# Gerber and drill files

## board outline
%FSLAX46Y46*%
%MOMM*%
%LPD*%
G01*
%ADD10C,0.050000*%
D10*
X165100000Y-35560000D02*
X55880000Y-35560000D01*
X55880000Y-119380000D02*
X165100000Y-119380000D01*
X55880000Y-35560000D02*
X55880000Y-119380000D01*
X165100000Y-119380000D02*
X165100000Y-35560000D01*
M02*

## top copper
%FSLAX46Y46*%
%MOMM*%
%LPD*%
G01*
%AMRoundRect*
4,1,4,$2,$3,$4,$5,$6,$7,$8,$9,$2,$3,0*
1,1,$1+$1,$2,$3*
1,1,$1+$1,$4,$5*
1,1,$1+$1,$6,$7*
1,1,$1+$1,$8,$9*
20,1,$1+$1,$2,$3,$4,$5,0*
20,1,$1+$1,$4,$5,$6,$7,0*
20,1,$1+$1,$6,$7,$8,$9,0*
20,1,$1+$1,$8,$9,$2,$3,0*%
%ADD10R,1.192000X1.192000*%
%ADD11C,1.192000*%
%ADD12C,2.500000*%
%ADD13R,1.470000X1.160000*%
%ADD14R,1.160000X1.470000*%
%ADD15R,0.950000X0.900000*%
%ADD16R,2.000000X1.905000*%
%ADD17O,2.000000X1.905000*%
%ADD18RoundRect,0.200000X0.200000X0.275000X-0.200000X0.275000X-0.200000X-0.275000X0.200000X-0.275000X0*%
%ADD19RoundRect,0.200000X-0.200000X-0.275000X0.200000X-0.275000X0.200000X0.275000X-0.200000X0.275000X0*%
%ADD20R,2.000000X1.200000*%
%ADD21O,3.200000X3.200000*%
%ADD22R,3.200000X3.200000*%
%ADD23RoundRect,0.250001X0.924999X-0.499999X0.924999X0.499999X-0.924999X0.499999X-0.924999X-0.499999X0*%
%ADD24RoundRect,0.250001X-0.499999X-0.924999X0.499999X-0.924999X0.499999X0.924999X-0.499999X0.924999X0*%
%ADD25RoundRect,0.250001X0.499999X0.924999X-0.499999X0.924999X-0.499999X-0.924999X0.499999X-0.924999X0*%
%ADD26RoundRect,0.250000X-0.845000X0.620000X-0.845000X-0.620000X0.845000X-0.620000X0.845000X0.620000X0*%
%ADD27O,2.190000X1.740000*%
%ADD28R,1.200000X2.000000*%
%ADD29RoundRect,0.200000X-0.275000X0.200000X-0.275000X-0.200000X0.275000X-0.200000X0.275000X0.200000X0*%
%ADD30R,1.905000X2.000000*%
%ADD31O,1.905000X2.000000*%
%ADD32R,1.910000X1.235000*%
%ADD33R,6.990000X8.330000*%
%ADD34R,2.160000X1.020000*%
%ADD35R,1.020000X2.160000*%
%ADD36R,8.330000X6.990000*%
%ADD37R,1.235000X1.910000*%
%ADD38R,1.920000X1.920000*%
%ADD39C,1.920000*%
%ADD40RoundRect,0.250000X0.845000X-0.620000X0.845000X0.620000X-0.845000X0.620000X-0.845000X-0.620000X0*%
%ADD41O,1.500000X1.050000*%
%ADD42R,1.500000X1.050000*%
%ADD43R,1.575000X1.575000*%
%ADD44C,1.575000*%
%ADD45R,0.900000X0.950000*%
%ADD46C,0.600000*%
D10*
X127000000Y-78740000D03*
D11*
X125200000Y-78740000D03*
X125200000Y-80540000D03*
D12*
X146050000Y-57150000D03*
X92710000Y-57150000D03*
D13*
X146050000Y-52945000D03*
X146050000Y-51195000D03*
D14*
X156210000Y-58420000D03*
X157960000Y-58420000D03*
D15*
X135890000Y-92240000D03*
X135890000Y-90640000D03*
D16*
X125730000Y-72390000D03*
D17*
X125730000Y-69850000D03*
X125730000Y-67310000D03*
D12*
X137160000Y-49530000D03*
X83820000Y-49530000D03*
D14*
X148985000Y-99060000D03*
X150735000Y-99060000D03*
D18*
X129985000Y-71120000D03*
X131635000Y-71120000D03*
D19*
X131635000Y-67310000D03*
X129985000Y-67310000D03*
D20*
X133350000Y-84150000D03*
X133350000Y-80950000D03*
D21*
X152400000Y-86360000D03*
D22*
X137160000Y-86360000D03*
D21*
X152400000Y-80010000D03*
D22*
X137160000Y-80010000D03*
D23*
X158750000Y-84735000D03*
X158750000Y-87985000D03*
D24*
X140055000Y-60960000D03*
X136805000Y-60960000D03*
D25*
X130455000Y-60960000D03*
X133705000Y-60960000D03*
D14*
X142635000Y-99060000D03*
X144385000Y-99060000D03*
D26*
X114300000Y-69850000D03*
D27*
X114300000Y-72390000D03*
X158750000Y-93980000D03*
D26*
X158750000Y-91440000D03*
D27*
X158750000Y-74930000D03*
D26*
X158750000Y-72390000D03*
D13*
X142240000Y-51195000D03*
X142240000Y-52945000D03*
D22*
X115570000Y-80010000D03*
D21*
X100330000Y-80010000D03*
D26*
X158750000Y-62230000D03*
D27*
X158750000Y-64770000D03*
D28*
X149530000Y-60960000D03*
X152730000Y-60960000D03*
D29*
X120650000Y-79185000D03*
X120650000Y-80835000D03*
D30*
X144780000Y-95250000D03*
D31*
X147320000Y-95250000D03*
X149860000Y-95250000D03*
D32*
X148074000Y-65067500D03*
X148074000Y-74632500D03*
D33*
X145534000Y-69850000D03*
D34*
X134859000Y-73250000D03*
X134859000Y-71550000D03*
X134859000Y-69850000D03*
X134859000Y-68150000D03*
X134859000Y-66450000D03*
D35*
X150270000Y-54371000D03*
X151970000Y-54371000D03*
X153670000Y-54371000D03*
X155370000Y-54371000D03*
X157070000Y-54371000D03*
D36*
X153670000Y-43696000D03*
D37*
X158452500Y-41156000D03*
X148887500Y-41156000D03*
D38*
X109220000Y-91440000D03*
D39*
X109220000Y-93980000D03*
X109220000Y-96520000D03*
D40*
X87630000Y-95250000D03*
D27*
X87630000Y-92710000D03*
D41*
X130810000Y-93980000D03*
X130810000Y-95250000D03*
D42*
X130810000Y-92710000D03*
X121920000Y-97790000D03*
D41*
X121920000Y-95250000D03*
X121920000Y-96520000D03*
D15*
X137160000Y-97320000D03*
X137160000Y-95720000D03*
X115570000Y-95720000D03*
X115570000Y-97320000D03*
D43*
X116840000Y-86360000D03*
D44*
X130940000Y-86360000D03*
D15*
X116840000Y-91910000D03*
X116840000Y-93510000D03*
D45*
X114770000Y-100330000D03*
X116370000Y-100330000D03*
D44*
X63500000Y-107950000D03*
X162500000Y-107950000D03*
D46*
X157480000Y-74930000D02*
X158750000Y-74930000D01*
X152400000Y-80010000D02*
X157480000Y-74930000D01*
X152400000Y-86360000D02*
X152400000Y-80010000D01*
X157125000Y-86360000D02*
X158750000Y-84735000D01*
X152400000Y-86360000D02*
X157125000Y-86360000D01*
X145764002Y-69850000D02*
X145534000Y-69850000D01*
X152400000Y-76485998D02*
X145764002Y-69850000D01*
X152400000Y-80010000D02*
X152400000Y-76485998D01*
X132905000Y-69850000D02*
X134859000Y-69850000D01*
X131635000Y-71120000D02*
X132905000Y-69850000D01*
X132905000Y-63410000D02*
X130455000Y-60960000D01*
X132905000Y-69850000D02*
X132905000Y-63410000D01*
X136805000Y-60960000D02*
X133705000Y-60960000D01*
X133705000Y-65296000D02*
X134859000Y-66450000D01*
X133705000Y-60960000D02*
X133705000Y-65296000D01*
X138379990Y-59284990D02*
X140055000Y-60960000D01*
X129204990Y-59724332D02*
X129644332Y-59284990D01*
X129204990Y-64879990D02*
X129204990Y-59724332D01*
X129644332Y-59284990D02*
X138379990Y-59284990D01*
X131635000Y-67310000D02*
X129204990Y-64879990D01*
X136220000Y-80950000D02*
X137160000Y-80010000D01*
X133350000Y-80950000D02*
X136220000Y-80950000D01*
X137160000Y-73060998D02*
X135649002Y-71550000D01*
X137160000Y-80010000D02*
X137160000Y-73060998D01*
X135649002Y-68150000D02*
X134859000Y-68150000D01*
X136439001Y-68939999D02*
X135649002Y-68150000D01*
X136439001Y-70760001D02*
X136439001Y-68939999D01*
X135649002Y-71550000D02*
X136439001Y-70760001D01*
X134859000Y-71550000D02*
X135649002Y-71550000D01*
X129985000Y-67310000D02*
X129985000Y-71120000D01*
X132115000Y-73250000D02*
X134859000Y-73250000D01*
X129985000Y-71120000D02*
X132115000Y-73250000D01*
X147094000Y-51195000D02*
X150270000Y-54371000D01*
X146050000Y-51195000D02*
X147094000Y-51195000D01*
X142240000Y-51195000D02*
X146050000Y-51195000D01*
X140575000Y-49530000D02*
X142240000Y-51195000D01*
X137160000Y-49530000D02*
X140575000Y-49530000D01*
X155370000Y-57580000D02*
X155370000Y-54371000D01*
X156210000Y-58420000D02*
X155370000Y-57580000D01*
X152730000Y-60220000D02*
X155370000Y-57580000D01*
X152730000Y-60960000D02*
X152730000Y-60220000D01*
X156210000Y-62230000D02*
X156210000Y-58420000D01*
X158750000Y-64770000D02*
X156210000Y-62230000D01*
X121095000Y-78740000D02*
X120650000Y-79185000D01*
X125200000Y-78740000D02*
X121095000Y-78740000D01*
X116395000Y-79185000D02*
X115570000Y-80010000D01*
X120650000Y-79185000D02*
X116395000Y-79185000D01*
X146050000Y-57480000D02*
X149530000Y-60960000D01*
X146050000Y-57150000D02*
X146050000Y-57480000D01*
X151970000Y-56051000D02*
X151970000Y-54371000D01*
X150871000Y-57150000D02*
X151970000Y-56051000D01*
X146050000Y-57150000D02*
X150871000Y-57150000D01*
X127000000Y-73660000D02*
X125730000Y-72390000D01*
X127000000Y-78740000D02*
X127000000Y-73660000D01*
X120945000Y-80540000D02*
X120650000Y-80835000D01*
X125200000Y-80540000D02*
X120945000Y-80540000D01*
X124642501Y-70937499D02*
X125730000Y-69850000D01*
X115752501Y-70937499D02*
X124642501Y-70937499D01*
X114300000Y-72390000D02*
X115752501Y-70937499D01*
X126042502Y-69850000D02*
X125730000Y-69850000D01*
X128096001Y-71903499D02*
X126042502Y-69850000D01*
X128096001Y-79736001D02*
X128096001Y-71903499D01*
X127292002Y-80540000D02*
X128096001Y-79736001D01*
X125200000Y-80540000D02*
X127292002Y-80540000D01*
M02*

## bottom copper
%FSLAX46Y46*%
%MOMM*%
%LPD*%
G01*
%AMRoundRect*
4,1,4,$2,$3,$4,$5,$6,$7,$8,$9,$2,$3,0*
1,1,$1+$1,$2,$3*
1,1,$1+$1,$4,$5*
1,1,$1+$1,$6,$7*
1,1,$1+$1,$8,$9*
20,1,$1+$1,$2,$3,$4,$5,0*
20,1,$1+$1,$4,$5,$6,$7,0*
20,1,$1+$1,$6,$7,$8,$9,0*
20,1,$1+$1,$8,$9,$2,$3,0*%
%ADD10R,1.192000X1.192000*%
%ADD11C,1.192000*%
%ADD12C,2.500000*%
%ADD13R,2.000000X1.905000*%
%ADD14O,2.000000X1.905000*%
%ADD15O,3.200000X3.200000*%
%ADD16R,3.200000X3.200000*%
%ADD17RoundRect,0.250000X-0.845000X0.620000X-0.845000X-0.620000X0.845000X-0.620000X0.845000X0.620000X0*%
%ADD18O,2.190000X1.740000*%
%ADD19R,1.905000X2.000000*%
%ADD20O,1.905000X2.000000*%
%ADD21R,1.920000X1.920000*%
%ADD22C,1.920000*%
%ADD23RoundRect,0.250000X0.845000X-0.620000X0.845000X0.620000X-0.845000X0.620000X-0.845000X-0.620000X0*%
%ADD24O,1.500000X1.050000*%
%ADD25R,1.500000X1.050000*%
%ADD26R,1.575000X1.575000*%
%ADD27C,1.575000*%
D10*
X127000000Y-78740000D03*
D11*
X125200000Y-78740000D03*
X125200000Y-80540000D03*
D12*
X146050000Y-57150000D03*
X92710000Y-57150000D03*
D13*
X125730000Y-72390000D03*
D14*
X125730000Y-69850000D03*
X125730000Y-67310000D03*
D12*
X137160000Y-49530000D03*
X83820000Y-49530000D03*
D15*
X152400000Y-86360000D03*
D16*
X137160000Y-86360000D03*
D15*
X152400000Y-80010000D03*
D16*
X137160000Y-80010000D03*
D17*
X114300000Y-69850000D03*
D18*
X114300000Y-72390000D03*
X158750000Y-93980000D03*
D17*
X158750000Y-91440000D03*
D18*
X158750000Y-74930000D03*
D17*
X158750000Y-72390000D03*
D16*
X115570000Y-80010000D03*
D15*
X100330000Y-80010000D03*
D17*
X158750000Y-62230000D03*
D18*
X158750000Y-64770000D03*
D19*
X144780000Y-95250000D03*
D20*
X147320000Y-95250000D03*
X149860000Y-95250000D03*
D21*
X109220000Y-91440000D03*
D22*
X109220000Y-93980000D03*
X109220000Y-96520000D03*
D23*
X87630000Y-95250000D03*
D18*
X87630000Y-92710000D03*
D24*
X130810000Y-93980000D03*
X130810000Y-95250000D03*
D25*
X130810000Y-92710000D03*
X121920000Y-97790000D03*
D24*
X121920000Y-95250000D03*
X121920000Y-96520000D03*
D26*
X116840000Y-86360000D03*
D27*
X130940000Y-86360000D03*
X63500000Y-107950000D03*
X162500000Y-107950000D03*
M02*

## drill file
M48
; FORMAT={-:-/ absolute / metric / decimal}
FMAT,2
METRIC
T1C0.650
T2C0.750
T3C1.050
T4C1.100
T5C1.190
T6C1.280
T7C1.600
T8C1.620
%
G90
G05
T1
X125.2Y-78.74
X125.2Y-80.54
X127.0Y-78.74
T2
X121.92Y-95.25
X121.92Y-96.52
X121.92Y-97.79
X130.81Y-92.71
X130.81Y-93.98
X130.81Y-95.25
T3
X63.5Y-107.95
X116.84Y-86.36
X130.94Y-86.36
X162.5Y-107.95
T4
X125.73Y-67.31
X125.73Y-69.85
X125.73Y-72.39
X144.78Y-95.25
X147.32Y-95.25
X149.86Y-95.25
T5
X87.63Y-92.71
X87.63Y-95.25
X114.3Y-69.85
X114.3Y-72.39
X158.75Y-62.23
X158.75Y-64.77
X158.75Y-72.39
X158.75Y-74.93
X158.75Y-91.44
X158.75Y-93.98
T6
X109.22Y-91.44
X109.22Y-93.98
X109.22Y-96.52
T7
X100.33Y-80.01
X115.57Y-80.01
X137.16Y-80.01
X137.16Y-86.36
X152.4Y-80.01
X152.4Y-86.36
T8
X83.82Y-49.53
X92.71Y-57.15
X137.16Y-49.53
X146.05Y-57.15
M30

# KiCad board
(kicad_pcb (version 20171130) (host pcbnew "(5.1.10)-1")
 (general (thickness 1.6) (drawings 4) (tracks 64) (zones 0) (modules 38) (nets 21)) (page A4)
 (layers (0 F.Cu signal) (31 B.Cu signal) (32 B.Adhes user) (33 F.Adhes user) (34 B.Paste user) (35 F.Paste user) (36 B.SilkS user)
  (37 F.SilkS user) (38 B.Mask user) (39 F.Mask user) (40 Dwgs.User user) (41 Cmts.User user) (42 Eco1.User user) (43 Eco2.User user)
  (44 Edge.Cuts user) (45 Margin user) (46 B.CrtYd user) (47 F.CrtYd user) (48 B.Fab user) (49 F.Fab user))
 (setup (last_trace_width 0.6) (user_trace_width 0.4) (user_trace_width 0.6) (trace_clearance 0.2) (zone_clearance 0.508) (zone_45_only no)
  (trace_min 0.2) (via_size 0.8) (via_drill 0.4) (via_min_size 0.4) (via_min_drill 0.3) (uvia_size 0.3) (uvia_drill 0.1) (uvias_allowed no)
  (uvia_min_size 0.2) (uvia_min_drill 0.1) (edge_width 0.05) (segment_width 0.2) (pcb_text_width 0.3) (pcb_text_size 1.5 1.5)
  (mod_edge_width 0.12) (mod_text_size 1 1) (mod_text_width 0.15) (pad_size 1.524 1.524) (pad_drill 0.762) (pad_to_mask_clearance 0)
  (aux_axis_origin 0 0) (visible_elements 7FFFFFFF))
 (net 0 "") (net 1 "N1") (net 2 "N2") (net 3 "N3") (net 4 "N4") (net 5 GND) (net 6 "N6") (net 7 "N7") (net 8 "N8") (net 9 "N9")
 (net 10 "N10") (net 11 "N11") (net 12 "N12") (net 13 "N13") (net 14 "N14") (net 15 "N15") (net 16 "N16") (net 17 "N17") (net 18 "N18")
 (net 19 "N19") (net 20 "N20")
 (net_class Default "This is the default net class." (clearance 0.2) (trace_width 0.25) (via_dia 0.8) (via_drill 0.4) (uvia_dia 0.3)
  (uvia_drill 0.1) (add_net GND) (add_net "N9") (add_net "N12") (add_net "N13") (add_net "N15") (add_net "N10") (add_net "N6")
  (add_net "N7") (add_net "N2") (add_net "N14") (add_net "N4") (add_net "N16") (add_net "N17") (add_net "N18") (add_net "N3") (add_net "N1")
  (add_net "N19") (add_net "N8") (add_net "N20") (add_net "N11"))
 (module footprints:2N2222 (layer F.Cu) (at 127 78.74 180)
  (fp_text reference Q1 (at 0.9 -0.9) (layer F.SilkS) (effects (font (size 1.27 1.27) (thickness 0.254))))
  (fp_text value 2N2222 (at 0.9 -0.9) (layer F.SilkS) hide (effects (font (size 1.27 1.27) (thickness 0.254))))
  (pad 1 thru_hole rect (at 0 0 180) (size 1.192 1.192) (drill 0.65) (layers *.Cu *.Mask) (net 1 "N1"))
  (pad 2 thru_hole circle (at 1.8 0 180) (size 1.192 1.192) (drill 0.65) (layers *.Cu *.Mask) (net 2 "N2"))
  (pad 3 thru_hole circle (at 1.8 -1.8 180) (size 1.192 1.192) (drill 0.65) (layers *.Cu *.Mask) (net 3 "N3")))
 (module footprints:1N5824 (layer F.Cu) (at 119.38 57.15)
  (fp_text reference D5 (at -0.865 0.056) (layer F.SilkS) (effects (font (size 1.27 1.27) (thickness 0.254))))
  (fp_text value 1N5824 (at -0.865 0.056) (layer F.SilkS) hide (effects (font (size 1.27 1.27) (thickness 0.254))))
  (pad 1 thru_hole circle (at 26.67 0) (size 2.5 2.5) (drill 1.62) (layers *.Cu *.Mask) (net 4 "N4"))
  (pad 2 thru_hole circle (at -26.67 0) (size 2.5 2.5) (drill 1.62) (layers *.Cu *.Mask) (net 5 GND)))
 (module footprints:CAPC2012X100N (layer F.Cu) (at 146.05 52.07 270)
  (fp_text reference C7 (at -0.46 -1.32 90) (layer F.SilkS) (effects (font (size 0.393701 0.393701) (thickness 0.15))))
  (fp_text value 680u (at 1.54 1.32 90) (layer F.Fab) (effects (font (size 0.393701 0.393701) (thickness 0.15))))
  (pad 2 smd rect (at 0.875 0 270) (size 1.16 1.47) (layers F.Cu F.Paste F.Mask) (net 5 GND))
  (pad 1 smd rect (at -0.875 0 270) (size 1.16 1.47) (layers F.Cu F.Paste F.Mask) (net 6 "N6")))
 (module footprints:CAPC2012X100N (layer F.Cu) (at 157.085 58.42)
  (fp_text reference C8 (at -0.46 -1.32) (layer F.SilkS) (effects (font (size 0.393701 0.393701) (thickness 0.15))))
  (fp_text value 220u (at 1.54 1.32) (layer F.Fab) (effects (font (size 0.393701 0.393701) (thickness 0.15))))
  (pad 1 smd rect (at -0.875 0) (size 1.16 1.47) (layers F.Cu F.Paste F.Mask) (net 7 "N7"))
  (pad 2 smd rect (at 0.875 0) (size 1.16 1.47) (layers F.Cu F.Paste F.Mask) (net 5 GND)))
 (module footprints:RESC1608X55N (layer F.Cu) (at 135.89 91.44 90)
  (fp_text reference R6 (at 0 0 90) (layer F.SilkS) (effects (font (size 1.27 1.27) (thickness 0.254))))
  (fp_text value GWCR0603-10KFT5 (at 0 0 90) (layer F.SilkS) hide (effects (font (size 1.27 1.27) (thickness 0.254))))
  (pad 1 smd rect (at -0.8 0 90) (size 0.9 0.95) (layers F.Cu F.Paste F.Mask) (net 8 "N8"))
  (pad 2 smd rect (at 0.8 0 90) (size 0.9 0.95) (layers F.Cu F.Paste F.Mask) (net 5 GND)))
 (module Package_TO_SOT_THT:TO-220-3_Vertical (layer F.Cu) (at 125.73 72.39 90)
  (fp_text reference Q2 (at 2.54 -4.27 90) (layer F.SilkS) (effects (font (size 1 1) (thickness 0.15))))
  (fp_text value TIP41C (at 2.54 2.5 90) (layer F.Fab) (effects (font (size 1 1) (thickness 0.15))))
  (pad 1 thru_hole rect (at 0 0 90) (size 1.905 2) (drill 1.1) (layers *.Cu *.Mask) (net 1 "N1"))
  (pad 2 thru_hole oval (at 2.54 0 90) (size 1.905 2) (drill 1.1) (layers *.Cu *.Mask) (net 3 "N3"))
  (pad 3 thru_hole oval (at 5.08 0 90) (size 1.905 2) (drill 1.1) (layers *.Cu *.Mask) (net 6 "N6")))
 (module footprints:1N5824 (layer F.Cu) (at 110.49 49.53 180)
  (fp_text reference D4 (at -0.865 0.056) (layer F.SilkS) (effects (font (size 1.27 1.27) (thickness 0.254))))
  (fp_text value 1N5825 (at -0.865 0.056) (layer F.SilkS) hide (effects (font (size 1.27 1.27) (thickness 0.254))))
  (pad 2 thru_hole circle (at -26.67 0 180) (size 2.5 2.5) (drill 1.62) (layers *.Cu *.Mask) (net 6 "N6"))
  (pad 1 thru_hole circle (at 26.67 0 180) (size 2.5 2.5) (drill 1.62) (layers *.Cu *.Mask) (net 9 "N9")))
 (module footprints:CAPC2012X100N (layer F.Cu) (at 149.86 99.06 180)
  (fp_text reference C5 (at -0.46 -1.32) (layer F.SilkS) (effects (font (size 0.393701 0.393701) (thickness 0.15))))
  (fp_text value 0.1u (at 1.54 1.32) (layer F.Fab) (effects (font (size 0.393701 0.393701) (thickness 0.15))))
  (pad 2 smd rect (at 0.875 0 180) (size 1.16 1.47) (layers F.Cu F.Paste F.Mask) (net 5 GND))
  (pad 1 smd rect (at -0.875 0 180) (size 1.16 1.47) (layers F.Cu F.Paste F.Mask) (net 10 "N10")))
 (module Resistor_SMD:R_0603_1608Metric (layer F.Cu) (at 130.81 71.12 180)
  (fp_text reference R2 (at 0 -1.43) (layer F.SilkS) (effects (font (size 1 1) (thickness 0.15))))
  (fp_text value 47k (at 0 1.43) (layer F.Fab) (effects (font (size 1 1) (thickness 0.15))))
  (pad 2 smd roundrect (at 0.825 0 180) (size 0.8 0.95) (layers F.Cu F.Paste F.Mask) (roundrect_rratio 0.25) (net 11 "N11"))
  (pad 1 smd roundrect (at -0.825 0 180) (size 0.8 0.95) (layers F.Cu F.Paste F.Mask) (roundrect_rratio 0.25) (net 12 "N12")))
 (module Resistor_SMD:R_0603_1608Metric (layer F.Cu) (at 130.81 67.31)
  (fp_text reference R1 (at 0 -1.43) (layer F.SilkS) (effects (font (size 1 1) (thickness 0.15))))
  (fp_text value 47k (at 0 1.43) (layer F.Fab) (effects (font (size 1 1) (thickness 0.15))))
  (pad 2 smd roundrect (at 0.825 0) (size 0.8 0.95) (layers F.Cu F.Paste F.Mask) (roundrect_rratio 0.25) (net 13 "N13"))
  (pad 1 smd roundrect (at -0.825 0) (size 0.8 0.95) (layers F.Cu F.Paste F.Mask) (roundrect_rratio 0.25) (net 11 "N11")))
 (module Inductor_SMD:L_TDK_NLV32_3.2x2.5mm (layer F.Cu) (at 133.35 82.55 270)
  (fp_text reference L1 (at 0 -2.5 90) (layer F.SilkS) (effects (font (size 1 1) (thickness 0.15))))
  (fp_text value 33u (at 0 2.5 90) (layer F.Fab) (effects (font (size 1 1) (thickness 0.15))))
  (pad 2 smd rect (at 1.6 0 270) (size 1.2 2) (layers F.Cu F.Paste F.Mask) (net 5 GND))
  (pad 1 smd rect (at -1.6 0 270) (size 1.2 2) (layers F.Cu F.Paste F.Mask) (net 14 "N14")))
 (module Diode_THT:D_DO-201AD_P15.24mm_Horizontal (layer F.Cu) (at 137.16 86.36)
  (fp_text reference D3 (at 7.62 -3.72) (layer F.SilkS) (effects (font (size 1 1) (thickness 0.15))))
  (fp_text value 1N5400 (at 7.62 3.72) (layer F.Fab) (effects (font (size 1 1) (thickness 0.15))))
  (pad 2 thru_hole oval (at 15.24 0) (size 3.2 3.2) (drill 1.6) (layers *.Cu *.Mask) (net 12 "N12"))
  (pad 1 thru_hole rect (at 0 0) (size 3.2 3.2) (drill 1.6) (layers *.Cu *.Mask) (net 5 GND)))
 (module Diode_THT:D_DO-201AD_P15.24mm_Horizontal (layer F.Cu) (at 137.16 80.01)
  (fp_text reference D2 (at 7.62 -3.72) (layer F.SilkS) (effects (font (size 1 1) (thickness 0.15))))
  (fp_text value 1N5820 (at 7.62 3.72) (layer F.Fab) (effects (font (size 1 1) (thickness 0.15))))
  (pad 2 thru_hole oval (at 15.24 0) (size 3.2 3.2) (drill 1.6) (layers *.Cu *.Mask) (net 12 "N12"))
  (pad 1 thru_hole rect (at 0 0) (size 3.2 3.2) (drill 1.6) (layers *.Cu *.Mask) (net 14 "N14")))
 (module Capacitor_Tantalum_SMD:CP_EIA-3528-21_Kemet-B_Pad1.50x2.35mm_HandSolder (layer F.Cu) (at 158.75 86.36 90)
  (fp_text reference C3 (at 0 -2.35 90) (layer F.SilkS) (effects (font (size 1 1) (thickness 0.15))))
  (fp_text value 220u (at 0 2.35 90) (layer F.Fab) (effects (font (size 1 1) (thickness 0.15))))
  (pad 2 smd roundrect (at 1.625 0 90) (size 1.5 2.35) (layers F.Cu F.Paste F.Mask) (roundrect_rratio 0.166667) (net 12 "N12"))
  (pad 1 smd roundrect (at -1.625 0 90) (size 1.5 2.35) (layers F.Cu F.Paste F.Mask) (roundrect_rratio 0.166667) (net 5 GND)))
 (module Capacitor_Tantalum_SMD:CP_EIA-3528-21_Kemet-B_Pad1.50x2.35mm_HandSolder (layer F.Cu) (at 138.43 60.96)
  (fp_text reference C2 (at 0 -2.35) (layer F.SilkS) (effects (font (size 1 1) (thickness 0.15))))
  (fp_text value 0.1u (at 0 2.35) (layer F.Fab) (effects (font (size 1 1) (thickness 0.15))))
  (pad 2 smd roundrect (at 1.625 0) (size 1.5 2.35) (layers F.Cu F.Paste F.Mask) (roundrect_rratio 0.166667) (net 13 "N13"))
  (pad 1 smd roundrect (at -1.625 0) (size 1.5 2.35) (layers F.Cu F.Paste F.Mask) (roundrect_rratio 0.166667) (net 9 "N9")))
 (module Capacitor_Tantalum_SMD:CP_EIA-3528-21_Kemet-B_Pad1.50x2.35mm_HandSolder (layer F.Cu) (at 132.08 60.96 180)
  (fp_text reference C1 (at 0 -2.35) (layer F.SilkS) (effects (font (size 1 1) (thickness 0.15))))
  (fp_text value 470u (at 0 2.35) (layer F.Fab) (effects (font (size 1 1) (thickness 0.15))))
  (pad 2 smd roundrect (at 1.625 0 180) (size 1.5 2.35) (layers F.Cu F.Paste F.Mask) (roundrect_rratio 0.166667) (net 12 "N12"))
  (pad 1 smd roundrect (at -1.625 0 180) (size 1.5 2.35) (layers F.Cu F.Paste F.Mask) (roundrect_rratio 0.166667) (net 9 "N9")))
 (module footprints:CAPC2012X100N (layer F.Cu) (at 143.51 99.06)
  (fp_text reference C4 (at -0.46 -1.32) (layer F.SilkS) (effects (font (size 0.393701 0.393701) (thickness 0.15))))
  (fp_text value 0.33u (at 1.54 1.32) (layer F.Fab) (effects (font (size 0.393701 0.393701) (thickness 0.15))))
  (pad 1 smd rect (at -0.875 0) (size 1.16 1.47) (layers F.Cu F.Paste F.Mask) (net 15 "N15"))
  (pad 2 smd rect (at 0.875 0) (size 1.16 1.47) (layers F.Cu F.Paste F.Mask) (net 5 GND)))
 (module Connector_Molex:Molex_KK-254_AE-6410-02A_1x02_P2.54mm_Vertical (layer F.Cu) (at 114.3 69.85 270)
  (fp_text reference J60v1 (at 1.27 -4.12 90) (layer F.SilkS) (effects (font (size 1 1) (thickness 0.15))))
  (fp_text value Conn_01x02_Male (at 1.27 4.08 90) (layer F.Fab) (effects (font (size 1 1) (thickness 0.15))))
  (pad 1 thru_hole roundrect (at 0 0 270) (size 1.74 2.19) (drill 1.19) (layers *.Cu *.Mask) (roundrect_rratio 0.143678) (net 5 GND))
  (pad 2 thru_hole oval (at 2.54 0 270) (size 1.74 2.19) (drill 1.19) (layers *.Cu *.Mask) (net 3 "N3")))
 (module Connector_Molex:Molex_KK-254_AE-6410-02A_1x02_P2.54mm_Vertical (layer F.Cu) (at 158.75 91.44 270)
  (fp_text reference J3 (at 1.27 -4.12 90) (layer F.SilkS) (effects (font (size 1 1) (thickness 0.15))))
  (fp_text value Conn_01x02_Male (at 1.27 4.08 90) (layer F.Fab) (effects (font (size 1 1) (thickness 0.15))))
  (pad 2 thru_hole oval (at 2.54 0 270) (size 1.74 2.19) (drill 1.19) (layers *.Cu *.Mask) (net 10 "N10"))
  (pad 1 thru_hole roundrect (at 0 0 270) (size 1.74 2.19) (drill 1.19) (layers *.Cu *.Mask) (roundrect_rratio 0.143678) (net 5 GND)))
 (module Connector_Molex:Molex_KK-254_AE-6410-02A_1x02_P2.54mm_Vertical (layer F.Cu) (at 158.75 72.39 270)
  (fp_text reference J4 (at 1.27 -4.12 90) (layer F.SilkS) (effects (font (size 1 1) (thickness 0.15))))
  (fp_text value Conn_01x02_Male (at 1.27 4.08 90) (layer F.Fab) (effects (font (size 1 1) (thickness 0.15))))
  (pad 2 thru_hole oval (at 2.54 0 270) (size 1.74 2.19) (drill 1.19) (layers *.Cu *.Mask) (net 12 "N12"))
  (pad 1 thru_hole roundrect (at 0 0 270) (size 1.74 2.19) (drill 1.19) (layers *.Cu *.Mask) (roundrect_rratio 0.143678) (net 5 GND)))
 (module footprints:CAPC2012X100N (layer F.Cu) (at 142.24 52.07 270)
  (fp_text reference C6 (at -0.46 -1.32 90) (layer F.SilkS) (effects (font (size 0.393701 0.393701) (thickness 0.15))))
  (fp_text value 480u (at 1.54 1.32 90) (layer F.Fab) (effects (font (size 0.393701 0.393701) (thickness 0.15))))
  (pad 1 smd rect (at -0.875 0 270) (size 1.16 1.47) (layers F.Cu F.Paste F.Mask) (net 6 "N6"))
  (pad 2 smd rect (at 0.875 0 270) (size 1.16 1.47) (layers F.Cu F.Paste F.Mask) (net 5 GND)))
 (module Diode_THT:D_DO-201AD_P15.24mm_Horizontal (layer F.Cu) (at 115.57 80.01 180)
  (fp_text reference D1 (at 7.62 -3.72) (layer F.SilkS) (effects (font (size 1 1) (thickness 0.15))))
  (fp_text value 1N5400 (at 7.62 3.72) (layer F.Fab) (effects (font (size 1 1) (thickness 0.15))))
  (pad 1 thru_hole rect (at 0 0 180) (size 3.2 3.2) (drill 1.6) (layers *.Cu *.Mask) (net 2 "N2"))
  (pad 2 thru_hole oval (at 15.24 0 180) (size 3.2 3.2) (drill 1.6) (layers *.Cu *.Mask) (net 5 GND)))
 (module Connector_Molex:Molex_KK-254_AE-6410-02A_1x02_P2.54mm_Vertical (layer F.Cu) (at 158.75 62.23 270)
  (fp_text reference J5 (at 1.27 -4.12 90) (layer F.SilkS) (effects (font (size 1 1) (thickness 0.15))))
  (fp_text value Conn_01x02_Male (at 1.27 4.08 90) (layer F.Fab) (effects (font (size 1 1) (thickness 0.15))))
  (pad 1 thru_hole roundrect (at 0 0 270) (size 1.74 2.19) (drill 1.19) (layers *.Cu *.Mask) (roundrect_rratio 0.143678) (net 5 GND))
  (pad 2 thru_hole oval (at 2.54 0 270) (size 1.74 2.19) (drill 1.19) (layers *.Cu *.Mask) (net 7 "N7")))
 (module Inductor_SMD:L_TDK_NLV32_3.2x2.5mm (layer F.Cu) (at 151.13 60.96)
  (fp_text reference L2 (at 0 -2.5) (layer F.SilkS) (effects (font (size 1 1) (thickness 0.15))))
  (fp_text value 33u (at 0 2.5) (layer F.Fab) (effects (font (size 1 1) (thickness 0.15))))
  (pad 1 smd rect (at -1.6 0) (size 1.2 2) (layers F.Cu F.Paste F.Mask) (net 4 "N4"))
  (pad 2 smd rect (at 1.6 0) (size 1.2 2) (layers F.Cu F.Paste F.Mask) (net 7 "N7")))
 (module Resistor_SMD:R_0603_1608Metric (layer F.Cu) (at 120.65 80.01 270)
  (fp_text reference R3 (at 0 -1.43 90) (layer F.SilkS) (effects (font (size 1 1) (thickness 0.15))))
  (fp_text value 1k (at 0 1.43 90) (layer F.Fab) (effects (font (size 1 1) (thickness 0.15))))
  (pad 1 smd roundrect (at -0.825 0 270) (size 0.8 0.95) (layers F.Cu F.Paste F.Mask) (roundrect_rratio 0.25) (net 2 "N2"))
  (pad 2 smd roundrect (at 0.825 0 270) (size 0.8 0.95) (layers F.Cu F.Paste F.Mask) (roundrect_rratio 0.25) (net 3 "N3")))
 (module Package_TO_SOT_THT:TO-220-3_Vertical (layer F.Cu) (at 144.78 95.25)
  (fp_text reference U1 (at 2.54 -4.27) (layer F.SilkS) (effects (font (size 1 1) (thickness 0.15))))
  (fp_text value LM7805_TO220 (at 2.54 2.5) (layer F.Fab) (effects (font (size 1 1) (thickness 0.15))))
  (pad 1 thru_hole rect (at 0 0) (size 1.905 2) (drill 1.1) (layers *.Cu *.Mask) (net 15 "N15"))
  (pad 2 thru_hole oval (at 2.54 0) (size 1.905 2) (drill 1.1) (layers *.Cu *.Mask) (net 5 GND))
  (pad 3 thru_hole oval (at 5.08 0) (size 1.905 2) (drill 1.1) (layers *.Cu *.Mask) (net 10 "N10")))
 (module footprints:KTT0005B (layer F.Cu) (at 147.32 69.85 180)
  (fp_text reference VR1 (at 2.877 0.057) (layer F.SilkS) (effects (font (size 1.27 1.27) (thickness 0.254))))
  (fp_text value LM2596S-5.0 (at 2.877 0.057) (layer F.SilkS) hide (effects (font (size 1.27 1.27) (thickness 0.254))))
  (pad 8 smd rect (at -0.754 4.7825 270) (size 1.235 1.91) (layers F.Cu F.Paste F.Mask))
  (pad 7 smd rect (at -0.754 -4.7825 270) (size 1.235 1.91) (layers F.Cu F.Paste F.Mask))
  (pad 6 smd rect (at 1.786 0 180) (size 6.99 8.33) (layers F.Cu F.Paste F.Mask) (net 12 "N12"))
  (pad 5 smd rect (at 12.461 -3.4 270) (size 1.02 2.16) (layers F.Cu F.Paste F.Mask) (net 11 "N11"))
  (pad 4 smd rect (at 12.461 -1.7 270) (size 1.02 2.16) (layers F.Cu F.Paste F.Mask) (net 14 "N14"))
  (pad 3 smd rect (at 12.461 0 270) (size 1.02 2.16) (layers F.Cu F.Paste F.Mask) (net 12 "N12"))
  (pad 2 smd rect (at 12.461 1.7 270) (size 1.02 2.16) (layers F.Cu F.Paste F.Mask) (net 14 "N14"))
  (pad 1 smd rect (at 12.461 3.4 270) (size 1.02 2.16) (layers F.Cu F.Paste F.Mask) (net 9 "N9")))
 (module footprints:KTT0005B (layer F.Cu) (at 153.67 41.91 270)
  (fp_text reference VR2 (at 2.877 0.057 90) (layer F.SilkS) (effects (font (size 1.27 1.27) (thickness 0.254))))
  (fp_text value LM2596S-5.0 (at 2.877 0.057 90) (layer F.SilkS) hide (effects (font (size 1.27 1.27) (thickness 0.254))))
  (pad 1 smd rect (at 12.461 3.4) (size 1.02 2.16) (layers F.Cu F.Paste F.Mask) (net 6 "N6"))
  (pad 2 smd rect (at 12.461 1.7) (size 1.02 2.16) (layers F.Cu F.Paste F.Mask) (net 4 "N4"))
  (pad 3 smd rect (at 12.461 0) (size 1.02 2.16) (layers F.Cu F.Paste F.Mask) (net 5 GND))
  (pad 4 smd rect (at 12.461 -1.7) (size 1.02 2.16) (layers F.Cu F.Paste F.Mask) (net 7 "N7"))
  (pad 5 smd rect (at 12.461 -3.4) (size 1.02 2.16) (layers F.Cu F.Paste F.Mask) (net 5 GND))
  (pad 6 smd rect (at 1.786 0 270) (size 6.99 8.33) (layers F.Cu F.Paste F.Mask) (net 5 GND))
  (pad 7 smd rect (at -0.754 -4.7825) (size 1.235 1.91) (layers F.Cu F.Paste F.Mask))
  (pad 8 smd rect (at -0.754 4.7825) (size 1.235 1.91) (layers F.Cu F.Paste F.Mask)))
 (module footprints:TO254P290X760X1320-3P (layer F.Cu) (at 109.22 91.44 270)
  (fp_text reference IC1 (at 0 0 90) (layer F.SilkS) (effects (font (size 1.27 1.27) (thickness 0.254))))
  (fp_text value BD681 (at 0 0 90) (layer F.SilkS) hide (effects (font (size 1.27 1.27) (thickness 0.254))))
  (pad 1 thru_hole rect (at 0 0 270) (size 1.92 1.92) (drill 1.28) (layers *.Cu *.Mask) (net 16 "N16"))
  (pad 2 thru_hole circle (at 2.54 0 270) (size 1.92 1.92) (drill 1.28) (layers *.Cu *.Mask) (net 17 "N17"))
  (pad 3 thru_hole circle (at 5.08 0 270) (size 1.92 1.92) (drill 1.28) (layers *.Cu *.Mask) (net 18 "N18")))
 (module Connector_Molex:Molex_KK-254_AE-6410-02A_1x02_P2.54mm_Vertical (layer F.Cu) (at 87.63 95.25 90)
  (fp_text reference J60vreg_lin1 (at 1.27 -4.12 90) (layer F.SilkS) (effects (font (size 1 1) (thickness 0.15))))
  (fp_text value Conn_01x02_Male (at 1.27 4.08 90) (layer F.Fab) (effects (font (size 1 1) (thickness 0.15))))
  (pad 1 thru_hole roundrect (at 0 0 90) (size 1.74 2.19) (drill 1.19) (layers *.Cu *.Mask) (roundrect_rratio 0.143678) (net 5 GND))
  (pad 2 thru_hole oval (at 2.54 0 90) (size 1.74 2.19) (drill 1.19) (layers *.Cu *.Mask) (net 17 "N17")))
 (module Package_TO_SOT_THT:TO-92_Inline (layer F.Cu) (at 130.81 92.71 270)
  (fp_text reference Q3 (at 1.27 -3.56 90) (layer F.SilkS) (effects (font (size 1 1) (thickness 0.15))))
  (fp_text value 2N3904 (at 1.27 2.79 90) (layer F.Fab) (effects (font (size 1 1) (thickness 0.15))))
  (pad 2 thru_hole oval (at 1.27 0 270) (size 1.05 1.5) (drill 0.75) (layers *.Cu *.Mask) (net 8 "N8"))
  (pad 3 thru_hole oval (at 2.54 0 270) (size 1.05 1.5) (drill 0.75) (layers *.Cu *.Mask) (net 16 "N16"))
  (pad 1 thru_hole rect (at 0 0 270) (size 1.05 1.5) (drill 0.75) (layers *.Cu *.Mask) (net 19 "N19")))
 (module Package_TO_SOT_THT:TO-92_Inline (layer F.Cu) (at 121.92 97.79 90)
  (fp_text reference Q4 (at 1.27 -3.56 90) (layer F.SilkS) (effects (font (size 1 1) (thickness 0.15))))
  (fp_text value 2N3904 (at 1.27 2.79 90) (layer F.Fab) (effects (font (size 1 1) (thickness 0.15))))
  (pad 1 thru_hole rect (at 0 0 90) (size 1.05 1.5) (drill 0.75) (layers *.Cu *.Mask) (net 15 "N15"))
  (pad 3 thru_hole oval (at 2.54 0 90) (size 1.05 1.5) (drill 0.75) (layers *.Cu *.Mask) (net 16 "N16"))
  (pad 2 thru_hole oval (at 1.27 0 90) (size 1.05 1.5) (drill 0.75) (layers *.Cu *.Mask) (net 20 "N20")))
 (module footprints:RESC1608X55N (layer F.Cu) (at 137.16 96.52 90)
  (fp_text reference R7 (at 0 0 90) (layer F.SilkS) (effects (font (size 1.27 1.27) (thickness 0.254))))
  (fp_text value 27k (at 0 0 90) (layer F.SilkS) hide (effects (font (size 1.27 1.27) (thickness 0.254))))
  (pad 1 smd rect (at -0.8 0 90) (size 0.9 0.95) (layers F.Cu F.Paste F.Mask) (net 15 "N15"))
  (pad 2 smd rect (at 0.8 0 90) (size 0.9 0.95) (layers F.Cu F.Paste F.Mask) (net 8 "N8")))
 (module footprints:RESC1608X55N (layer F.Cu) (at 115.57 96.52 90)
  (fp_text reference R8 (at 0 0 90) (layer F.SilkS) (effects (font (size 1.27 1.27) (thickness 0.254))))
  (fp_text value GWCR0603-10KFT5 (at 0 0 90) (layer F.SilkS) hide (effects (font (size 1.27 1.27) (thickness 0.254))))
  (pad 2 smd rect (at 0.8 0 90) (size 0.9 0.95) (layers F.Cu F.Paste F.Mask) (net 18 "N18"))
  (pad 1 smd rect (at -0.8 0 90) (size 0.9 0.95) (layers F.Cu F.Paste F.Mask) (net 20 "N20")))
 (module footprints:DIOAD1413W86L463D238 (layer F.Cu) (at 116.84 86.36)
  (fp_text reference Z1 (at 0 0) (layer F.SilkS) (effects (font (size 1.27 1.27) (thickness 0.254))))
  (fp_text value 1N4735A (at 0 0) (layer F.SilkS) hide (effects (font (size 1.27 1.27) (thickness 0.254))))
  (pad 1 thru_hole rect (at 0 0) (size 1.575 1.575) (drill 1.05) (layers *.Cu *.Mask) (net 19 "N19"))
  (pad 2 thru_hole circle (at 14.1 0) (size 1.575 1.575) (drill 1.05) (layers *.Cu *.Mask) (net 5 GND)))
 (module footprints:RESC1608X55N (layer F.Cu) (at 116.84 92.71 90)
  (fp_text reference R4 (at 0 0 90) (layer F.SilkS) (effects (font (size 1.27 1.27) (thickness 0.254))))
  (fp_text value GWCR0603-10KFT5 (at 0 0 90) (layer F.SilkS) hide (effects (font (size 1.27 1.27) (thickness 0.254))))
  (pad 2 smd rect (at 0.8 0 90) (size 0.9 0.95) (layers F.Cu F.Paste F.Mask) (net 16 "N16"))
  (pad 1 smd rect (at -0.8 0 90) (size 0.9 0.95) (layers F.Cu F.Paste F.Mask) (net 17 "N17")))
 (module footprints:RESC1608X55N (layer F.Cu) (at 115.57 100.33)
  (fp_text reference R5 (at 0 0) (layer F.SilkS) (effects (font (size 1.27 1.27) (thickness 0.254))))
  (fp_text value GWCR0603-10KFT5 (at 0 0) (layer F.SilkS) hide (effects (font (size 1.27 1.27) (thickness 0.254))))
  (pad 1 smd rect (at -0.8 0) (size 0.9 0.95) (layers F.Cu F.Paste F.Mask) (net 5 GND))
  (pad 2 smd rect (at 0.8 0) (size 0.9 0.95) (layers F.Cu F.Paste F.Mask) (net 20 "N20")))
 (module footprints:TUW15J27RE (layer F.Cu) (at 63.5 107.95)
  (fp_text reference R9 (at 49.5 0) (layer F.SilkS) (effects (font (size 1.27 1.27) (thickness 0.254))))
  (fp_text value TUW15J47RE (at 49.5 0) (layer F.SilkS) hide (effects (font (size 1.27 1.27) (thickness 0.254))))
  (pad 1 thru_hole circle (at 0 0) (size 1.575 1.575) (drill 1.05) (layers *.Cu *.Mask) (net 18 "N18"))
  (pad 2 thru_hole circle (at 99 0) (size 1.575 1.575) (drill 1.05) (layers *.Cu *.Mask) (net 15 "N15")))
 (gr_line (start 165.1 35.56) (end 55.88 35.56) (layer Edge.Cuts) (width 0.05))
 (gr_line (start 55.88 119.38) (end 165.1 119.38) (layer Edge.Cuts) (width 0.05))
 (gr_line (start 55.88 35.56) (end 55.88 119.38) (layer Edge.Cuts) (width 0.05))
 (gr_line (start 165.1 119.38) (end 165.1 35.56) (layer Edge.Cuts) (width 0.05))
 (segment (start 157.48 74.93) (end 158.75 74.93) (width 0.6) (layer F.Cu) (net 12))
 (segment (start 152.4 80.01) (end 157.48 74.93) (width 0.6) (layer F.Cu) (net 12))
 (segment (start 152.4 86.36) (end 152.4 80.01) (width 0.6) (layer F.Cu) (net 12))
 (segment (start 157.125 86.36) (end 158.75 84.735) (width 0.6) (layer F.Cu) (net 12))
 (segment (start 152.4 86.36) (end 157.125 86.36) (width 0.6) (layer F.Cu) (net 12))
 (segment (start 145.764002 69.85) (end 145.534 69.85) (width 0.6) (layer F.Cu) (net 12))
 (segment (start 152.4 76.485998) (end 145.764002 69.85) (width 0.6) (layer F.Cu) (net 12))
 (segment (start 152.4 80.01) (end 152.4 76.485998) (width 0.6) (layer F.Cu) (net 12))
 (segment (start 132.905 69.85) (end 134.859 69.85) (width 0.6) (layer F.Cu) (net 12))
 (segment (start 131.635 71.12) (end 132.905 69.85) (width 0.6) (layer F.Cu) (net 12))
 (segment (start 132.905 63.41) (end 130.455 60.96) (width 0.6) (layer F.Cu) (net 12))
 (segment (start 132.905 69.85) (end 132.905 63.41) (width 0.6) (layer F.Cu) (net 12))
 (segment (start 136.805 60.96) (end 133.705 60.96) (width 0.6) (layer F.Cu) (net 9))
 (segment (start 133.705 65.296) (end 134.859 66.45) (width 0.6) (layer F.Cu) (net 9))
 (segment (start 133.705 60.96) (end 133.705 65.296) (width 0.6) (layer F.Cu) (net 9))
 (segment (start 138.37999 59.28499) (end 140.055 60.96) (width 0.6) (layer F.Cu) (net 13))
 (segment (start 129.20499 59.724332) (end 129.644332 59.28499) (width 0.6) (layer F.Cu) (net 13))
 (segment (start 129.20499 64.87999) (end 129.20499 59.724332) (width 0.6) (layer F.Cu) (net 13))
 (segment (start 129.644332 59.28499) (end 138.37999 59.28499) (width 0.6) (layer F.Cu) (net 13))
 (segment (start 131.635 67.31) (end 129.20499 64.87999) (width 0.6) (layer F.Cu) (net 13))
 (segment (start 136.22 80.95) (end 137.16 80.01) (width 0.6) (layer F.Cu) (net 14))
 (segment (start 133.35 80.95) (end 136.22 80.95) (width 0.6) (layer F.Cu) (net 14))
 (segment (start 137.16 73.060998) (end 135.649002 71.55) (width 0.6) (layer F.Cu) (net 14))
 (segment (start 137.16 80.01) (end 137.16 73.060998) (width 0.6) (layer F.Cu) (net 14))
 (segment (start 135.649002 68.15) (end 134.859 68.15) (width 0.6) (layer F.Cu) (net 14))
 (segment (start 136.439001 68.939999) (end 135.649002 68.15) (width 0.6) (layer F.Cu) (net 14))
 (segment (start 136.439001 70.760001) (end 136.439001 68.939999) (width 0.6) (layer F.Cu) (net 14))
 (segment (start 135.649002 71.55) (end 136.439001 70.760001) (width 0.6) (layer F.Cu) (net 14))
 (segment (start 134.859 71.55) (end 135.649002 71.55) (width 0.6) (layer F.Cu) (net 14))
 (segment (start 129.985 67.31) (end 129.985 71.12) (width 0.6) (layer F.Cu) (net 11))
 (segment (start 132.115 73.25) (end 134.859 73.25) (width 0.6) (layer F.Cu) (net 11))
 (segment (start 129.985 71.12) (end 132.115 73.25) (width 0.6) (layer F.Cu) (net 11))
 (segment (start 147.094 51.195) (end 150.27 54.371) (width 0.6) (layer F.Cu) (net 6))
 (segment (start 146.05 51.195) (end 147.094 51.195) (width 0.6) (layer F.Cu) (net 6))
 (segment (start 142.24 51.195) (end 146.05 51.195) (width 0.6) (layer F.Cu) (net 6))
 (segment (start 140.575 49.53) (end 142.24 51.195) (width 0.6) (layer F.Cu) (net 6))
 (segment (start 137.16 49.53) (end 140.575 49.53) (width 0.6) (layer F.Cu) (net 6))
 (segment (start 155.37 57.58) (end 155.37 54.371) (width 0.6) (layer F.Cu) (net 7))
 (segment (start 156.21 58.42) (end 155.37 57.58) (width 0.6) (layer F.Cu) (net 7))
 (segment (start 152.73 60.22) (end 155.37 57.58) (width 0.6) (layer F.Cu) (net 7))
 (segment (start 152.73 60.96) (end 152.73 60.22) (width 0.6) (layer F.Cu) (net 7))
 (segment (start 156.21 62.23) (end 156.21 58.42) (width 0.6) (layer F.Cu) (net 7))
 (segment (start 158.75 64.77) (end 156.21 62.23) (width 0.6) (layer F.Cu) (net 7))
 (segment (start 121.095 78.74) (end 120.65 79.185) (width 0.6) (layer F.Cu) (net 2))
 (segment (start 125.2 78.74) (end 121.095 78.74) (width 0.6) (layer F.Cu) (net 2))
 (segment (start 116.395 79.185) (end 115.57 80.01) (width 0.6) (layer F.Cu) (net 2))
 (segment (start 120.65 79.185) (end 116.395 79.185) (width 0.6) (layer F.Cu) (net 2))
 (segment (start 146.05 57.48) (end 149.53 60.96) (width 0.6) (layer F.Cu) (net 4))
 (segment (start 146.05 57.15) (end 146.05 57.48) (width 0.6) (layer F.Cu) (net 4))
 (segment (start 151.97 56.051) (end 151.97 54.371) (width 0.6) (layer F.Cu) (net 4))
 (segment (start 150.871 57.15) (end 151.97 56.051) (width 0.6) (layer F.Cu) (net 4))
 (segment (start 146.05 57.15) (end 150.871 57.15) (width 0.6) (layer F.Cu) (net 4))
 (segment (start 127 73.66) (end 125.73 72.39) (width 0.6) (layer F.Cu) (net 1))
 (segment (start 127 78.74) (end 127 73.66) (width 0.6) (layer F.Cu) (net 1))
 (segment (start 120.945 80.54) (end 120.65 80.835) (width 0.6) (layer F.Cu) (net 3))
 (segment (start 125.2 80.54) (end 120.945 80.54) (width 0.6) (layer F.Cu) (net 3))
 (segment (start 124.642501 70.937499) (end 125.73 69.85) (width 0.6) (layer F.Cu) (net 3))
 (segment (start 115.752501 70.937499) (end 124.642501 70.937499) (width 0.6) (layer F.Cu) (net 3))
 (segment (start 114.3 72.39) (end 115.752501 70.937499) (width 0.6) (layer F.Cu) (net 3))
 (segment (start 126.042502 69.85) (end 125.73 69.85) (width 0.6) (layer F.Cu) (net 3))
 (segment (start 128.096001 71.903499) (end 126.042502 69.85) (width 0.6) (layer F.Cu) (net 3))
 (segment (start 128.096001 79.736001) (end 128.096001 71.903499) (width 0.6) (layer F.Cu) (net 3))
 (segment (start 127.292002 80.54) (end 128.096001 79.736001) (width 0.6) (layer F.Cu) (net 3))
 (segment (start 125.2 80.54) (end 127.292002 80.54) (width 0.6) (layer F.Cu) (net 3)))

